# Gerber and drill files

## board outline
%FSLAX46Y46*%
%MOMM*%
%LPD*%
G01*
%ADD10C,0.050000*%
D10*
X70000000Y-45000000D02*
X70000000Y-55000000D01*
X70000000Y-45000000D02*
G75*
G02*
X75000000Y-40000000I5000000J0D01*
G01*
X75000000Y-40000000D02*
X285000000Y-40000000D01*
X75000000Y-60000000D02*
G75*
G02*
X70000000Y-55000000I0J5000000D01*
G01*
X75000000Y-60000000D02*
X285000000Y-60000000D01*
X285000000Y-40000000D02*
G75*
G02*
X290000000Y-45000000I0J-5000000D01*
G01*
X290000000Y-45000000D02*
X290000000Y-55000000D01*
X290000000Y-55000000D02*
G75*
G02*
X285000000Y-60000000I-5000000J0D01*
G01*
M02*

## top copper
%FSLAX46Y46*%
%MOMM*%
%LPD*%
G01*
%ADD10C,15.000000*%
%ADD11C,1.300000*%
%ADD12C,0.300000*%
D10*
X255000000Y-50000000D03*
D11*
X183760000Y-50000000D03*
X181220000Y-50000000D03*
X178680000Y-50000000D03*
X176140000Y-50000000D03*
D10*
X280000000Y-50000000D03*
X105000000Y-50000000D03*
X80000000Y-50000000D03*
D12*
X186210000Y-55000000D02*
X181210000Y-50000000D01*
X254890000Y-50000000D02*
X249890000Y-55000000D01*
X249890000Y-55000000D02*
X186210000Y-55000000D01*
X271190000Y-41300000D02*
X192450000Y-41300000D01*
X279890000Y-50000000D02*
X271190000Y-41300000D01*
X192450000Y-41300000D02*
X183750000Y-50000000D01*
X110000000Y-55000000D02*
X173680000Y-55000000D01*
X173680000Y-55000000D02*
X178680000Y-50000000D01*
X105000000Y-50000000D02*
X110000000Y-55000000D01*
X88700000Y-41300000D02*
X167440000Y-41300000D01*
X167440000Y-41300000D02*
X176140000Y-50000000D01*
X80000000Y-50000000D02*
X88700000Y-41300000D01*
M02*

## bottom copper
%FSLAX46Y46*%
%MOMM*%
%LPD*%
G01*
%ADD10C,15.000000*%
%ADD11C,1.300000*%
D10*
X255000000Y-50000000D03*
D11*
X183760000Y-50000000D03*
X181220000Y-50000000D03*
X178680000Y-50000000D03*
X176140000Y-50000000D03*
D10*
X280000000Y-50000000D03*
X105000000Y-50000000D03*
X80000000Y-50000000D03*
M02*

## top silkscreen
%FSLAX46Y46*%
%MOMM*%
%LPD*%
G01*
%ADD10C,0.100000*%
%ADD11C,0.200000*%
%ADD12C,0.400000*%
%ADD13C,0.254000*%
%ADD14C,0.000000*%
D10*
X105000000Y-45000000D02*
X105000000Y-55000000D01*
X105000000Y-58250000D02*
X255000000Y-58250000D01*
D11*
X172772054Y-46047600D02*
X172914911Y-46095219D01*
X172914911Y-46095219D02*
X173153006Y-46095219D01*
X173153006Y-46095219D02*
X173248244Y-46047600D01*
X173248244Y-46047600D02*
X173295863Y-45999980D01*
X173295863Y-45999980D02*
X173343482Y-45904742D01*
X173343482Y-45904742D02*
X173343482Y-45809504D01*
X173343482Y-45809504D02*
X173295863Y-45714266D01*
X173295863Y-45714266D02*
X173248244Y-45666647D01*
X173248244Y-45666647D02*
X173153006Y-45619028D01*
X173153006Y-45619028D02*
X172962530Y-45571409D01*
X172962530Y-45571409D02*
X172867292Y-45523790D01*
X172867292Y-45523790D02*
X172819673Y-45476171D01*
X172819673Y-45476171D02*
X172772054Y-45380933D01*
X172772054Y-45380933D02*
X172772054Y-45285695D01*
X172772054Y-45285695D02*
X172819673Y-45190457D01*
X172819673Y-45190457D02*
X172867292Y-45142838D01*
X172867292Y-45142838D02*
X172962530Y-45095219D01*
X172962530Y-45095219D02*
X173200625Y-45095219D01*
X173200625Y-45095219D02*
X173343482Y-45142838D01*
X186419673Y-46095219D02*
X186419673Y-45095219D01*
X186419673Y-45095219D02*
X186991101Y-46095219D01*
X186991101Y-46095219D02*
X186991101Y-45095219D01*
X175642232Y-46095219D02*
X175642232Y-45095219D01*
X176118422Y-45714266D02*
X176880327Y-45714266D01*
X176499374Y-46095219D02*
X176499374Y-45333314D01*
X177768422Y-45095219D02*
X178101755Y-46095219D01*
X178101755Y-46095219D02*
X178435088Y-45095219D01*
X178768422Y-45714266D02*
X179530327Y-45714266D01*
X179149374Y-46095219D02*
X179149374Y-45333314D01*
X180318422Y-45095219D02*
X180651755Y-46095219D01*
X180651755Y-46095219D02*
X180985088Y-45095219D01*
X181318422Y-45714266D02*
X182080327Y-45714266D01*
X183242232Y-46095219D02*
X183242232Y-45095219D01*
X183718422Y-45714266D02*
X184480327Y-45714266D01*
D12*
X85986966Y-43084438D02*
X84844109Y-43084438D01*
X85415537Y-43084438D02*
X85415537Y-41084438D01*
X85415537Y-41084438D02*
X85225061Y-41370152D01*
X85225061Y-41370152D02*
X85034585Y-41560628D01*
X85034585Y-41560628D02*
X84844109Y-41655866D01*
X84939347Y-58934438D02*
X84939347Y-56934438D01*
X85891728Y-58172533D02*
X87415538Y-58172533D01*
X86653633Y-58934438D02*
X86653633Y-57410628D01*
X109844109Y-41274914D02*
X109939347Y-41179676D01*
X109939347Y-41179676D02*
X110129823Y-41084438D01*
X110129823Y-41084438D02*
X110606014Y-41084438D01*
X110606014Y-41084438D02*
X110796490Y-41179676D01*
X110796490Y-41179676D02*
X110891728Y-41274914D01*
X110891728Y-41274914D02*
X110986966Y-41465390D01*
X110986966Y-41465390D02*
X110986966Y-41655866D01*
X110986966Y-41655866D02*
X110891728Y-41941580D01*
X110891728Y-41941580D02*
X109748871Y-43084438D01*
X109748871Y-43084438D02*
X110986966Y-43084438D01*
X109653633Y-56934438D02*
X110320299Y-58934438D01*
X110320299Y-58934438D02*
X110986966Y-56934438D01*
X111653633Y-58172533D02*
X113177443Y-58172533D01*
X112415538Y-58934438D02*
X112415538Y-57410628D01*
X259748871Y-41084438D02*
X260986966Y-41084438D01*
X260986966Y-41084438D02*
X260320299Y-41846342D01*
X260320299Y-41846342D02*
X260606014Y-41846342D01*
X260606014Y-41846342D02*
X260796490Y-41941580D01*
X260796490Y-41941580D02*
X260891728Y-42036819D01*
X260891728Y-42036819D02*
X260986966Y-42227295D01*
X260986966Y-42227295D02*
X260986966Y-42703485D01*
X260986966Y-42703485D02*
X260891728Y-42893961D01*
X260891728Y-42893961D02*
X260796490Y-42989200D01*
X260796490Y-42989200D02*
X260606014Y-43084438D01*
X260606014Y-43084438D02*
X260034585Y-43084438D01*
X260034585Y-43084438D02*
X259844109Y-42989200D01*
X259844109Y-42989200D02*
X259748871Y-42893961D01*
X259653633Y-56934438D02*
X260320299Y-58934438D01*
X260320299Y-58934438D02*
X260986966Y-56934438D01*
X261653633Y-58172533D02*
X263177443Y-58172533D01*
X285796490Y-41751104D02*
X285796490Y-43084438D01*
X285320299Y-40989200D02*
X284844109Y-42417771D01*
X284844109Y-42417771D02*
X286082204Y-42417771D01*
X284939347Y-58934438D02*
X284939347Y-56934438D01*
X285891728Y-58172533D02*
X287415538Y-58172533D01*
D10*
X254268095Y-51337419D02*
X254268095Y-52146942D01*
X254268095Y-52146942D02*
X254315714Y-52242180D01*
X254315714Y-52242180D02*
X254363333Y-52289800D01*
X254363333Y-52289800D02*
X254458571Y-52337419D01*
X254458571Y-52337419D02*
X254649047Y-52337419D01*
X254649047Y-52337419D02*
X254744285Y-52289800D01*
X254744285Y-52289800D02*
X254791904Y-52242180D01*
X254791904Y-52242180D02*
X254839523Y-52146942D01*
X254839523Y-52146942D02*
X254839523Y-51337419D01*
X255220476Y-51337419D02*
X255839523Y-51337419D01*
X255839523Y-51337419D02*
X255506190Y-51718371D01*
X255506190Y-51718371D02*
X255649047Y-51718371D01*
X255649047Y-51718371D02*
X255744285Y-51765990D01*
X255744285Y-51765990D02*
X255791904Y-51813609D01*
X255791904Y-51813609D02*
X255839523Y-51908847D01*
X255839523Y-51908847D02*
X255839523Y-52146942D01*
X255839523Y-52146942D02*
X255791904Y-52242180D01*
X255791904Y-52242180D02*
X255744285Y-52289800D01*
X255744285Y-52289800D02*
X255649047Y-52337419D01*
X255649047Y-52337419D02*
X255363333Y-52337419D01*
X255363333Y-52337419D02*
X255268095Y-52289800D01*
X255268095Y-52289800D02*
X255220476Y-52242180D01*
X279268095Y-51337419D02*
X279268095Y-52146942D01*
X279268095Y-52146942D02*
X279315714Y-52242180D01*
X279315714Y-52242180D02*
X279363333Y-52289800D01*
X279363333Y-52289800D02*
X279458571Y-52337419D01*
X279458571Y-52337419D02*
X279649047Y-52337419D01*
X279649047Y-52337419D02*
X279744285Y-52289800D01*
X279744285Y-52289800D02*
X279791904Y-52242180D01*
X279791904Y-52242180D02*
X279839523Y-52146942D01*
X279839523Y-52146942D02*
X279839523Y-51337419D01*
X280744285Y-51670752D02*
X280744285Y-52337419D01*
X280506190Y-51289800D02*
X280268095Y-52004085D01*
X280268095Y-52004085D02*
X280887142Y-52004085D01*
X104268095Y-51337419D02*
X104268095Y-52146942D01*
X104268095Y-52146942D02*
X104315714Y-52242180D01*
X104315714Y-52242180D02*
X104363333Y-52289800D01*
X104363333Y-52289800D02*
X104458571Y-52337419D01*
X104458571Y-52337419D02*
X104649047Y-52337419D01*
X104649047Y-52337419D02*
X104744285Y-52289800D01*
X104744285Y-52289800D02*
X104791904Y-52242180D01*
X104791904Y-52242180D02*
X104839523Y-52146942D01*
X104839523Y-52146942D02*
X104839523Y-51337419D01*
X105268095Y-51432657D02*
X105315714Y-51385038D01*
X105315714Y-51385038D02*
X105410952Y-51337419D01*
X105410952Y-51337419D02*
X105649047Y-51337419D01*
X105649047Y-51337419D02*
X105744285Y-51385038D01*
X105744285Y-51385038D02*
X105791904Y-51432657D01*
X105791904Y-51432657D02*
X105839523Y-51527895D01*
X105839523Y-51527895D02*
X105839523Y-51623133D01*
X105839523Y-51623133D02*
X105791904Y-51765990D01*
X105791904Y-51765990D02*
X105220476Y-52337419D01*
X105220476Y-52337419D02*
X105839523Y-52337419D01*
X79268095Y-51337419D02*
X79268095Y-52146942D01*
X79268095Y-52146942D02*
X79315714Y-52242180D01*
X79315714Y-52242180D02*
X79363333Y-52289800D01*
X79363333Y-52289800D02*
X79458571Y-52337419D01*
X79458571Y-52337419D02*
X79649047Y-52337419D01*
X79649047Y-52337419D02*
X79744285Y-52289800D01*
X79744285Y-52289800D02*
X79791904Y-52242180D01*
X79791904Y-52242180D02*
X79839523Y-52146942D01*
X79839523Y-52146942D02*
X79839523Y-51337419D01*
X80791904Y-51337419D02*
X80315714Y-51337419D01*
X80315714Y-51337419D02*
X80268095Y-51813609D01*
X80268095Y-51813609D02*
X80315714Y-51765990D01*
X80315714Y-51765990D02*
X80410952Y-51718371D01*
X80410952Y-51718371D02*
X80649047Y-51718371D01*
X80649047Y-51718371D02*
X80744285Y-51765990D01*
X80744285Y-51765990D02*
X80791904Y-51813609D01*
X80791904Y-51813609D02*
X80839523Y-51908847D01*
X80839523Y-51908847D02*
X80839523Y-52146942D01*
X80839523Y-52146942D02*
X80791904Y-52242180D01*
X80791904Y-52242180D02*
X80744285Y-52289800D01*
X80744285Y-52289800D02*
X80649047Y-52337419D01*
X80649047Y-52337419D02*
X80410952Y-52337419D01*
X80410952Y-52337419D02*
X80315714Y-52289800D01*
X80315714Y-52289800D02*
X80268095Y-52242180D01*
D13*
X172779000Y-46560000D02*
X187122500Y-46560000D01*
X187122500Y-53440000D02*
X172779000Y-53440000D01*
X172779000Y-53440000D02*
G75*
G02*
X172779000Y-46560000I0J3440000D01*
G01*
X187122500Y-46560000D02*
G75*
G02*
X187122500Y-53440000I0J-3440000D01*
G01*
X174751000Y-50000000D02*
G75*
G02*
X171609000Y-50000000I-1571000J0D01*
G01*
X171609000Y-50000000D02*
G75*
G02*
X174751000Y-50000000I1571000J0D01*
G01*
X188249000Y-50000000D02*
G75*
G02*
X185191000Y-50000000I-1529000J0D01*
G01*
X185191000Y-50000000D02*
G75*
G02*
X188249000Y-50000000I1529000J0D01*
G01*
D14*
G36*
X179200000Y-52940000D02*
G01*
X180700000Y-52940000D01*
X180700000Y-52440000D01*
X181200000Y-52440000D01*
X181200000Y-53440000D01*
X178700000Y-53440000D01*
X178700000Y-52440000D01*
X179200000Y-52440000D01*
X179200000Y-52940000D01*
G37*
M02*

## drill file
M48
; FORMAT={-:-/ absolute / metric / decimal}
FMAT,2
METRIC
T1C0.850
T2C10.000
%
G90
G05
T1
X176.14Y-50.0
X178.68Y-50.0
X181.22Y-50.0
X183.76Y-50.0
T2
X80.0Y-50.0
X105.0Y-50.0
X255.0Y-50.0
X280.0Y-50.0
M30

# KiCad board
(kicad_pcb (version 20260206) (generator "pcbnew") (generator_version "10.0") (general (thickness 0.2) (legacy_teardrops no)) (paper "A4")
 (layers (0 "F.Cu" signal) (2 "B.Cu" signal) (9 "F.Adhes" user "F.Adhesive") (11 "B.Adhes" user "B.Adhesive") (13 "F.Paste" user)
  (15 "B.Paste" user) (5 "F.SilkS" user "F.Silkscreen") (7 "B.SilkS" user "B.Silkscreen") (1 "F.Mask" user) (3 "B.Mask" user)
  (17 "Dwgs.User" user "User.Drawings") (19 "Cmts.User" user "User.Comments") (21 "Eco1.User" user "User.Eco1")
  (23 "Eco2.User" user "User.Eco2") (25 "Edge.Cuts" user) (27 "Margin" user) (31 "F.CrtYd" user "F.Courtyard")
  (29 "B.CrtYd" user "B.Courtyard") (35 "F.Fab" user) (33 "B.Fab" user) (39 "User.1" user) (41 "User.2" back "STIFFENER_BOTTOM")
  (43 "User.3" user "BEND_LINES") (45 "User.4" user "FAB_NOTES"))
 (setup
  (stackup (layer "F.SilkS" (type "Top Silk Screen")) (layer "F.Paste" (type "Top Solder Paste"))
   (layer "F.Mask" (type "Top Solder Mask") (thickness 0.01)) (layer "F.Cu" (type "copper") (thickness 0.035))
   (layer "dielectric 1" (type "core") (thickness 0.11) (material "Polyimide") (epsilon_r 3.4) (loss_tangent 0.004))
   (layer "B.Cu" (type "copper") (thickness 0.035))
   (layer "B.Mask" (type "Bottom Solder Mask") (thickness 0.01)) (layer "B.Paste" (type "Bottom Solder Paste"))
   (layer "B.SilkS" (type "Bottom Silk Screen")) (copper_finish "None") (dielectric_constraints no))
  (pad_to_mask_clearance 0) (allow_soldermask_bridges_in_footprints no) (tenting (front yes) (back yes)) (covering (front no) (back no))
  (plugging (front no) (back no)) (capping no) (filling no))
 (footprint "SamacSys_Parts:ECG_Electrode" (layer "F.Cu") (at 255.03 52.38)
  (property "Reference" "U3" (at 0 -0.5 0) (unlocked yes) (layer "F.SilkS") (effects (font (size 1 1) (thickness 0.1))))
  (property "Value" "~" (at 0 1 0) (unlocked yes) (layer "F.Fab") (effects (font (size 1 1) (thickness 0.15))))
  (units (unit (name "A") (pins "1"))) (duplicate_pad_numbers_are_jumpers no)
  (pad "1" thru_hole circle (at -0.03 -2.38) (size 15 15) (drill 10) (layers "*.Cu" "*.Mask") (remove_unused_layers no) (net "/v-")))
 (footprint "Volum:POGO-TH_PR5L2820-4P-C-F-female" (layer "F.Cu") (at 179.95 50 180)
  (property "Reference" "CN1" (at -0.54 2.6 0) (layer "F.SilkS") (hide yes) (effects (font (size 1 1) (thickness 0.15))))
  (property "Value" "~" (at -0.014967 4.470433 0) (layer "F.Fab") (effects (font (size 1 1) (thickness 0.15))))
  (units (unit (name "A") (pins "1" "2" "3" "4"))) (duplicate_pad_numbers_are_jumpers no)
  (fp_line (start 7.171 3.44) (end -7.1725 3.44) (stroke (width 0.254) (type default)) (layer "F.SilkS"))
  (fp_line (start -7.1725 -3.44) (end 7.171 -3.44) (stroke (width 0.254) (type default)) (layer "F.SilkS"))
  (fp_arc (start 7.171 -3.44) (mid 10.611 0) (end 7.171 3.44) (stroke (width 0.254) (type default)) (layer "F.SilkS"))
  (fp_arc (start -7.1725 3.44) (mid -10.6125 0) (end -7.1725 -3.44) (stroke (width 0.254) (type default)) (layer "F.SilkS"))
  (fp_circle (center 6.77 0) (end 8.341 0) (stroke (width 0.254) (type default)) (fill no) (layer "F.SilkS"))
  (fp_circle (center -6.77 0) (end -5.241 0) (stroke (width 0.254) (type default)) (fill no) (layer "F.SilkS"))
  (fp_poly
   (pts (xy 1.25 -2.44) (xy 1.25 -3.44) (xy -1.25 -3.44) (xy -1.25 -2.44) (xy -0.75 -2.44) (xy -0.75 -2.94) (xy 0.75 -2.94) (xy 0.75 -2.44))
   (stroke (width 0) (type default)) (fill yes) (layer "F.SilkS"))
  (pad "1" thru_hole circle (at -3.81 0 180) (size 1.3 1.3) (drill 0.85) (layers "*.Cu" "*.Mask") (remove_unused_layers no) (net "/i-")
   (thermal_bridge_angle 90))
  (pad "2" thru_hole circle (at -1.27 0 180) (size 1.3 1.3) (drill 0.85) (layers "*.Cu" "*.Mask") (remove_unused_layers no) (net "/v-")
   (thermal_bridge_angle 90))
  (pad "3" thru_hole circle (at 1.27 0 180) (size 1.3 1.3) (drill 0.85) (layers "*.Cu" "*.Mask") (remove_unused_layers no) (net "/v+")
   (thermal_bridge_angle 90))
  (pad "4" thru_hole circle (at 3.81 0 180) (size 1.3 1.3) (drill 0.85) (layers "*.Cu" "*.Mask") (remove_unused_layers no) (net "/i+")
   (thermal_bridge_angle 90)))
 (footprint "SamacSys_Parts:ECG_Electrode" (layer "F.Cu") (at 280.03 52.38)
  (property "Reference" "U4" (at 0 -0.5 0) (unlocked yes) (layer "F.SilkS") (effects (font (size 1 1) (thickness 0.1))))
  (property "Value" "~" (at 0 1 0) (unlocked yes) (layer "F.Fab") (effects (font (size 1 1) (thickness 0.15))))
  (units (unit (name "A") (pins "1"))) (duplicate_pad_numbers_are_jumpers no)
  (pad "1" thru_hole circle (at -0.03 -2.38) (size 15 15) (drill 10) (layers "*.Cu" "*.Mask") (remove_unused_layers no) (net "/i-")))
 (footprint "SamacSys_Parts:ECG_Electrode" (layer "F.Cu") (at 105.03 52.38)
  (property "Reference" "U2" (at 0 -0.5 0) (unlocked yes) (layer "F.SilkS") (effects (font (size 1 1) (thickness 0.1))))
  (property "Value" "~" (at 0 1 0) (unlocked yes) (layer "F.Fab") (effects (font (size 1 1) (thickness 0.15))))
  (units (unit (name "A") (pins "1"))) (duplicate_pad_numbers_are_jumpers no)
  (pad "1" thru_hole circle (at -0.03 -2.38) (size 15 15) (drill 10) (layers "*.Cu" "*.Mask") (remove_unused_layers no) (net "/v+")))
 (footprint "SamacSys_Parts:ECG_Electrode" (layer "F.Cu") (at 80.03 52.38)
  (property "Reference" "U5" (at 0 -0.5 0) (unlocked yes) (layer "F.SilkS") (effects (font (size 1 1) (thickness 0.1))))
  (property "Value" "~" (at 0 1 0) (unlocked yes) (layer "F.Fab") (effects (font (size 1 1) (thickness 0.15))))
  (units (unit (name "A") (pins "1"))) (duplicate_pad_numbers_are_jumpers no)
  (pad "1" thru_hole circle (at -0.03 -2.38) (size 15 15) (drill 10) (layers "*.Cu" "*.Mask") (remove_unused_layers no) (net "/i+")))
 (gr_line (start 105 45) (end 105 55) (stroke (width 0.1) (type default)) (layer "F.SilkS"))
 (gr_line (start 105 58.25) (end 255 58.25) (stroke (width 0.1) (type default)) (layer "F.SilkS"))
 (gr_line (start 70 45) (end 70 55) (stroke (width 0.05) (type default)) (layer "Edge.Cuts"))
 (gr_arc (start 70 45) (mid 71.464466 41.464466) (end 75 40) (stroke (width 0.05) (type default)) (layer "Edge.Cuts"))
 (gr_line (start 75 40) (end 285 40) (stroke (width 0.05) (type default)) (layer "Edge.Cuts"))
 (gr_arc (start 75 60) (mid 71.464466 58.535534) (end 70 55) (stroke (width 0.05) (type default)) (layer "Edge.Cuts"))
 (gr_line (start 75 60) (end 285 60) (stroke (width 0.05) (type default)) (layer "Edge.Cuts"))
 (gr_arc (start 285 40) (mid 288.535534 41.464466) (end 290 45) (stroke (width 0.05) (type default)) (layer "Edge.Cuts"))
 (gr_line (start 290 45) (end 290 55) (stroke (width 0.05) (type default)) (layer "Edge.Cuts"))
 (gr_arc (start 290 55) (mid 288.535534 58.535534) (end 285 60) (stroke (width 0.05) (type default)) (layer "Edge.Cuts"))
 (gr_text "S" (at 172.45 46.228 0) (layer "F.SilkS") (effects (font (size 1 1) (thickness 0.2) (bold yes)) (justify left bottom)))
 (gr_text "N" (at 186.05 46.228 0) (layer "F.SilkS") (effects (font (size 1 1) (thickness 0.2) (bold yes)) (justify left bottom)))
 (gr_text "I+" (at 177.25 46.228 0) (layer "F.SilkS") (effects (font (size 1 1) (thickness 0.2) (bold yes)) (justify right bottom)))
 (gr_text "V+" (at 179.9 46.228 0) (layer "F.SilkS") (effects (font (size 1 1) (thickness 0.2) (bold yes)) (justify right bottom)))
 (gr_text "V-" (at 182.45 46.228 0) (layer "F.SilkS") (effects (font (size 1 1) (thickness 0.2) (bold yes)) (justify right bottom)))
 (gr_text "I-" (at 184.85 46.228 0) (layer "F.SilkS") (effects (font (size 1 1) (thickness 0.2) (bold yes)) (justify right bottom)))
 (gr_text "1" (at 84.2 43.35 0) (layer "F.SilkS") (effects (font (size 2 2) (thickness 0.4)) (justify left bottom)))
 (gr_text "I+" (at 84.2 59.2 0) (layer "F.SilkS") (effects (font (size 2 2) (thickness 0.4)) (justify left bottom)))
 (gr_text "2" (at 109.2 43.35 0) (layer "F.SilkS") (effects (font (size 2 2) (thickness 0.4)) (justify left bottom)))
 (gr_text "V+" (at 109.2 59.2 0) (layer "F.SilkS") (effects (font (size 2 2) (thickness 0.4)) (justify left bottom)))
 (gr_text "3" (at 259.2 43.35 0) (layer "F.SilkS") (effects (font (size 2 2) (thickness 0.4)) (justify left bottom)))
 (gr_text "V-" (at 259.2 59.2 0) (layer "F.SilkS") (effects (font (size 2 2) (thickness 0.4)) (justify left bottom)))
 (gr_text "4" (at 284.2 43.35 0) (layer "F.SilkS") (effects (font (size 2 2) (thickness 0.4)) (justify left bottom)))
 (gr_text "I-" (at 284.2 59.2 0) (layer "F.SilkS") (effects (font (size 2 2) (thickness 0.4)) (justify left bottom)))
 (segment (start 186.21 55) (end 181.21 50) (width 0.3) (layer "F.Cu") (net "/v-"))
 (segment (start 254.89 50) (end 249.89 55) (width 0.3) (layer "F.Cu") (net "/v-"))
 (segment (start 249.89 55) (end 186.21 55) (width 0.3) (layer "F.Cu") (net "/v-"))
 (segment (start 271.19 41.3) (end 192.45 41.3) (width 0.3) (layer "F.Cu") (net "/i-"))
 (segment (start 279.89 50) (end 271.19 41.3) (width 0.3) (layer "F.Cu") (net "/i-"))
 (segment (start 192.45 41.3) (end 183.75 50) (width 0.3) (layer "F.Cu") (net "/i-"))
 (segment (start 110 55) (end 173.68 55) (width 0.3) (layer "F.Cu") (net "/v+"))
 (segment (start 173.68 55) (end 178.68 50) (width 0.3) (layer "F.Cu") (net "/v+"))
 (segment (start 105 50) (end 110 55) (width 0.3) (layer "F.Cu") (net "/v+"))
 (segment (start 88.7 41.3) (end 167.44 41.3) (width 0.3) (layer "F.Cu") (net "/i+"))
 (segment (start 167.44 41.3) (end 176.14 50) (width 0.3) (layer "F.Cu") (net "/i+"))
 (segment (start 80 50) (end 88.7 41.3) (width 0.3) (layer "F.Cu") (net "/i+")))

